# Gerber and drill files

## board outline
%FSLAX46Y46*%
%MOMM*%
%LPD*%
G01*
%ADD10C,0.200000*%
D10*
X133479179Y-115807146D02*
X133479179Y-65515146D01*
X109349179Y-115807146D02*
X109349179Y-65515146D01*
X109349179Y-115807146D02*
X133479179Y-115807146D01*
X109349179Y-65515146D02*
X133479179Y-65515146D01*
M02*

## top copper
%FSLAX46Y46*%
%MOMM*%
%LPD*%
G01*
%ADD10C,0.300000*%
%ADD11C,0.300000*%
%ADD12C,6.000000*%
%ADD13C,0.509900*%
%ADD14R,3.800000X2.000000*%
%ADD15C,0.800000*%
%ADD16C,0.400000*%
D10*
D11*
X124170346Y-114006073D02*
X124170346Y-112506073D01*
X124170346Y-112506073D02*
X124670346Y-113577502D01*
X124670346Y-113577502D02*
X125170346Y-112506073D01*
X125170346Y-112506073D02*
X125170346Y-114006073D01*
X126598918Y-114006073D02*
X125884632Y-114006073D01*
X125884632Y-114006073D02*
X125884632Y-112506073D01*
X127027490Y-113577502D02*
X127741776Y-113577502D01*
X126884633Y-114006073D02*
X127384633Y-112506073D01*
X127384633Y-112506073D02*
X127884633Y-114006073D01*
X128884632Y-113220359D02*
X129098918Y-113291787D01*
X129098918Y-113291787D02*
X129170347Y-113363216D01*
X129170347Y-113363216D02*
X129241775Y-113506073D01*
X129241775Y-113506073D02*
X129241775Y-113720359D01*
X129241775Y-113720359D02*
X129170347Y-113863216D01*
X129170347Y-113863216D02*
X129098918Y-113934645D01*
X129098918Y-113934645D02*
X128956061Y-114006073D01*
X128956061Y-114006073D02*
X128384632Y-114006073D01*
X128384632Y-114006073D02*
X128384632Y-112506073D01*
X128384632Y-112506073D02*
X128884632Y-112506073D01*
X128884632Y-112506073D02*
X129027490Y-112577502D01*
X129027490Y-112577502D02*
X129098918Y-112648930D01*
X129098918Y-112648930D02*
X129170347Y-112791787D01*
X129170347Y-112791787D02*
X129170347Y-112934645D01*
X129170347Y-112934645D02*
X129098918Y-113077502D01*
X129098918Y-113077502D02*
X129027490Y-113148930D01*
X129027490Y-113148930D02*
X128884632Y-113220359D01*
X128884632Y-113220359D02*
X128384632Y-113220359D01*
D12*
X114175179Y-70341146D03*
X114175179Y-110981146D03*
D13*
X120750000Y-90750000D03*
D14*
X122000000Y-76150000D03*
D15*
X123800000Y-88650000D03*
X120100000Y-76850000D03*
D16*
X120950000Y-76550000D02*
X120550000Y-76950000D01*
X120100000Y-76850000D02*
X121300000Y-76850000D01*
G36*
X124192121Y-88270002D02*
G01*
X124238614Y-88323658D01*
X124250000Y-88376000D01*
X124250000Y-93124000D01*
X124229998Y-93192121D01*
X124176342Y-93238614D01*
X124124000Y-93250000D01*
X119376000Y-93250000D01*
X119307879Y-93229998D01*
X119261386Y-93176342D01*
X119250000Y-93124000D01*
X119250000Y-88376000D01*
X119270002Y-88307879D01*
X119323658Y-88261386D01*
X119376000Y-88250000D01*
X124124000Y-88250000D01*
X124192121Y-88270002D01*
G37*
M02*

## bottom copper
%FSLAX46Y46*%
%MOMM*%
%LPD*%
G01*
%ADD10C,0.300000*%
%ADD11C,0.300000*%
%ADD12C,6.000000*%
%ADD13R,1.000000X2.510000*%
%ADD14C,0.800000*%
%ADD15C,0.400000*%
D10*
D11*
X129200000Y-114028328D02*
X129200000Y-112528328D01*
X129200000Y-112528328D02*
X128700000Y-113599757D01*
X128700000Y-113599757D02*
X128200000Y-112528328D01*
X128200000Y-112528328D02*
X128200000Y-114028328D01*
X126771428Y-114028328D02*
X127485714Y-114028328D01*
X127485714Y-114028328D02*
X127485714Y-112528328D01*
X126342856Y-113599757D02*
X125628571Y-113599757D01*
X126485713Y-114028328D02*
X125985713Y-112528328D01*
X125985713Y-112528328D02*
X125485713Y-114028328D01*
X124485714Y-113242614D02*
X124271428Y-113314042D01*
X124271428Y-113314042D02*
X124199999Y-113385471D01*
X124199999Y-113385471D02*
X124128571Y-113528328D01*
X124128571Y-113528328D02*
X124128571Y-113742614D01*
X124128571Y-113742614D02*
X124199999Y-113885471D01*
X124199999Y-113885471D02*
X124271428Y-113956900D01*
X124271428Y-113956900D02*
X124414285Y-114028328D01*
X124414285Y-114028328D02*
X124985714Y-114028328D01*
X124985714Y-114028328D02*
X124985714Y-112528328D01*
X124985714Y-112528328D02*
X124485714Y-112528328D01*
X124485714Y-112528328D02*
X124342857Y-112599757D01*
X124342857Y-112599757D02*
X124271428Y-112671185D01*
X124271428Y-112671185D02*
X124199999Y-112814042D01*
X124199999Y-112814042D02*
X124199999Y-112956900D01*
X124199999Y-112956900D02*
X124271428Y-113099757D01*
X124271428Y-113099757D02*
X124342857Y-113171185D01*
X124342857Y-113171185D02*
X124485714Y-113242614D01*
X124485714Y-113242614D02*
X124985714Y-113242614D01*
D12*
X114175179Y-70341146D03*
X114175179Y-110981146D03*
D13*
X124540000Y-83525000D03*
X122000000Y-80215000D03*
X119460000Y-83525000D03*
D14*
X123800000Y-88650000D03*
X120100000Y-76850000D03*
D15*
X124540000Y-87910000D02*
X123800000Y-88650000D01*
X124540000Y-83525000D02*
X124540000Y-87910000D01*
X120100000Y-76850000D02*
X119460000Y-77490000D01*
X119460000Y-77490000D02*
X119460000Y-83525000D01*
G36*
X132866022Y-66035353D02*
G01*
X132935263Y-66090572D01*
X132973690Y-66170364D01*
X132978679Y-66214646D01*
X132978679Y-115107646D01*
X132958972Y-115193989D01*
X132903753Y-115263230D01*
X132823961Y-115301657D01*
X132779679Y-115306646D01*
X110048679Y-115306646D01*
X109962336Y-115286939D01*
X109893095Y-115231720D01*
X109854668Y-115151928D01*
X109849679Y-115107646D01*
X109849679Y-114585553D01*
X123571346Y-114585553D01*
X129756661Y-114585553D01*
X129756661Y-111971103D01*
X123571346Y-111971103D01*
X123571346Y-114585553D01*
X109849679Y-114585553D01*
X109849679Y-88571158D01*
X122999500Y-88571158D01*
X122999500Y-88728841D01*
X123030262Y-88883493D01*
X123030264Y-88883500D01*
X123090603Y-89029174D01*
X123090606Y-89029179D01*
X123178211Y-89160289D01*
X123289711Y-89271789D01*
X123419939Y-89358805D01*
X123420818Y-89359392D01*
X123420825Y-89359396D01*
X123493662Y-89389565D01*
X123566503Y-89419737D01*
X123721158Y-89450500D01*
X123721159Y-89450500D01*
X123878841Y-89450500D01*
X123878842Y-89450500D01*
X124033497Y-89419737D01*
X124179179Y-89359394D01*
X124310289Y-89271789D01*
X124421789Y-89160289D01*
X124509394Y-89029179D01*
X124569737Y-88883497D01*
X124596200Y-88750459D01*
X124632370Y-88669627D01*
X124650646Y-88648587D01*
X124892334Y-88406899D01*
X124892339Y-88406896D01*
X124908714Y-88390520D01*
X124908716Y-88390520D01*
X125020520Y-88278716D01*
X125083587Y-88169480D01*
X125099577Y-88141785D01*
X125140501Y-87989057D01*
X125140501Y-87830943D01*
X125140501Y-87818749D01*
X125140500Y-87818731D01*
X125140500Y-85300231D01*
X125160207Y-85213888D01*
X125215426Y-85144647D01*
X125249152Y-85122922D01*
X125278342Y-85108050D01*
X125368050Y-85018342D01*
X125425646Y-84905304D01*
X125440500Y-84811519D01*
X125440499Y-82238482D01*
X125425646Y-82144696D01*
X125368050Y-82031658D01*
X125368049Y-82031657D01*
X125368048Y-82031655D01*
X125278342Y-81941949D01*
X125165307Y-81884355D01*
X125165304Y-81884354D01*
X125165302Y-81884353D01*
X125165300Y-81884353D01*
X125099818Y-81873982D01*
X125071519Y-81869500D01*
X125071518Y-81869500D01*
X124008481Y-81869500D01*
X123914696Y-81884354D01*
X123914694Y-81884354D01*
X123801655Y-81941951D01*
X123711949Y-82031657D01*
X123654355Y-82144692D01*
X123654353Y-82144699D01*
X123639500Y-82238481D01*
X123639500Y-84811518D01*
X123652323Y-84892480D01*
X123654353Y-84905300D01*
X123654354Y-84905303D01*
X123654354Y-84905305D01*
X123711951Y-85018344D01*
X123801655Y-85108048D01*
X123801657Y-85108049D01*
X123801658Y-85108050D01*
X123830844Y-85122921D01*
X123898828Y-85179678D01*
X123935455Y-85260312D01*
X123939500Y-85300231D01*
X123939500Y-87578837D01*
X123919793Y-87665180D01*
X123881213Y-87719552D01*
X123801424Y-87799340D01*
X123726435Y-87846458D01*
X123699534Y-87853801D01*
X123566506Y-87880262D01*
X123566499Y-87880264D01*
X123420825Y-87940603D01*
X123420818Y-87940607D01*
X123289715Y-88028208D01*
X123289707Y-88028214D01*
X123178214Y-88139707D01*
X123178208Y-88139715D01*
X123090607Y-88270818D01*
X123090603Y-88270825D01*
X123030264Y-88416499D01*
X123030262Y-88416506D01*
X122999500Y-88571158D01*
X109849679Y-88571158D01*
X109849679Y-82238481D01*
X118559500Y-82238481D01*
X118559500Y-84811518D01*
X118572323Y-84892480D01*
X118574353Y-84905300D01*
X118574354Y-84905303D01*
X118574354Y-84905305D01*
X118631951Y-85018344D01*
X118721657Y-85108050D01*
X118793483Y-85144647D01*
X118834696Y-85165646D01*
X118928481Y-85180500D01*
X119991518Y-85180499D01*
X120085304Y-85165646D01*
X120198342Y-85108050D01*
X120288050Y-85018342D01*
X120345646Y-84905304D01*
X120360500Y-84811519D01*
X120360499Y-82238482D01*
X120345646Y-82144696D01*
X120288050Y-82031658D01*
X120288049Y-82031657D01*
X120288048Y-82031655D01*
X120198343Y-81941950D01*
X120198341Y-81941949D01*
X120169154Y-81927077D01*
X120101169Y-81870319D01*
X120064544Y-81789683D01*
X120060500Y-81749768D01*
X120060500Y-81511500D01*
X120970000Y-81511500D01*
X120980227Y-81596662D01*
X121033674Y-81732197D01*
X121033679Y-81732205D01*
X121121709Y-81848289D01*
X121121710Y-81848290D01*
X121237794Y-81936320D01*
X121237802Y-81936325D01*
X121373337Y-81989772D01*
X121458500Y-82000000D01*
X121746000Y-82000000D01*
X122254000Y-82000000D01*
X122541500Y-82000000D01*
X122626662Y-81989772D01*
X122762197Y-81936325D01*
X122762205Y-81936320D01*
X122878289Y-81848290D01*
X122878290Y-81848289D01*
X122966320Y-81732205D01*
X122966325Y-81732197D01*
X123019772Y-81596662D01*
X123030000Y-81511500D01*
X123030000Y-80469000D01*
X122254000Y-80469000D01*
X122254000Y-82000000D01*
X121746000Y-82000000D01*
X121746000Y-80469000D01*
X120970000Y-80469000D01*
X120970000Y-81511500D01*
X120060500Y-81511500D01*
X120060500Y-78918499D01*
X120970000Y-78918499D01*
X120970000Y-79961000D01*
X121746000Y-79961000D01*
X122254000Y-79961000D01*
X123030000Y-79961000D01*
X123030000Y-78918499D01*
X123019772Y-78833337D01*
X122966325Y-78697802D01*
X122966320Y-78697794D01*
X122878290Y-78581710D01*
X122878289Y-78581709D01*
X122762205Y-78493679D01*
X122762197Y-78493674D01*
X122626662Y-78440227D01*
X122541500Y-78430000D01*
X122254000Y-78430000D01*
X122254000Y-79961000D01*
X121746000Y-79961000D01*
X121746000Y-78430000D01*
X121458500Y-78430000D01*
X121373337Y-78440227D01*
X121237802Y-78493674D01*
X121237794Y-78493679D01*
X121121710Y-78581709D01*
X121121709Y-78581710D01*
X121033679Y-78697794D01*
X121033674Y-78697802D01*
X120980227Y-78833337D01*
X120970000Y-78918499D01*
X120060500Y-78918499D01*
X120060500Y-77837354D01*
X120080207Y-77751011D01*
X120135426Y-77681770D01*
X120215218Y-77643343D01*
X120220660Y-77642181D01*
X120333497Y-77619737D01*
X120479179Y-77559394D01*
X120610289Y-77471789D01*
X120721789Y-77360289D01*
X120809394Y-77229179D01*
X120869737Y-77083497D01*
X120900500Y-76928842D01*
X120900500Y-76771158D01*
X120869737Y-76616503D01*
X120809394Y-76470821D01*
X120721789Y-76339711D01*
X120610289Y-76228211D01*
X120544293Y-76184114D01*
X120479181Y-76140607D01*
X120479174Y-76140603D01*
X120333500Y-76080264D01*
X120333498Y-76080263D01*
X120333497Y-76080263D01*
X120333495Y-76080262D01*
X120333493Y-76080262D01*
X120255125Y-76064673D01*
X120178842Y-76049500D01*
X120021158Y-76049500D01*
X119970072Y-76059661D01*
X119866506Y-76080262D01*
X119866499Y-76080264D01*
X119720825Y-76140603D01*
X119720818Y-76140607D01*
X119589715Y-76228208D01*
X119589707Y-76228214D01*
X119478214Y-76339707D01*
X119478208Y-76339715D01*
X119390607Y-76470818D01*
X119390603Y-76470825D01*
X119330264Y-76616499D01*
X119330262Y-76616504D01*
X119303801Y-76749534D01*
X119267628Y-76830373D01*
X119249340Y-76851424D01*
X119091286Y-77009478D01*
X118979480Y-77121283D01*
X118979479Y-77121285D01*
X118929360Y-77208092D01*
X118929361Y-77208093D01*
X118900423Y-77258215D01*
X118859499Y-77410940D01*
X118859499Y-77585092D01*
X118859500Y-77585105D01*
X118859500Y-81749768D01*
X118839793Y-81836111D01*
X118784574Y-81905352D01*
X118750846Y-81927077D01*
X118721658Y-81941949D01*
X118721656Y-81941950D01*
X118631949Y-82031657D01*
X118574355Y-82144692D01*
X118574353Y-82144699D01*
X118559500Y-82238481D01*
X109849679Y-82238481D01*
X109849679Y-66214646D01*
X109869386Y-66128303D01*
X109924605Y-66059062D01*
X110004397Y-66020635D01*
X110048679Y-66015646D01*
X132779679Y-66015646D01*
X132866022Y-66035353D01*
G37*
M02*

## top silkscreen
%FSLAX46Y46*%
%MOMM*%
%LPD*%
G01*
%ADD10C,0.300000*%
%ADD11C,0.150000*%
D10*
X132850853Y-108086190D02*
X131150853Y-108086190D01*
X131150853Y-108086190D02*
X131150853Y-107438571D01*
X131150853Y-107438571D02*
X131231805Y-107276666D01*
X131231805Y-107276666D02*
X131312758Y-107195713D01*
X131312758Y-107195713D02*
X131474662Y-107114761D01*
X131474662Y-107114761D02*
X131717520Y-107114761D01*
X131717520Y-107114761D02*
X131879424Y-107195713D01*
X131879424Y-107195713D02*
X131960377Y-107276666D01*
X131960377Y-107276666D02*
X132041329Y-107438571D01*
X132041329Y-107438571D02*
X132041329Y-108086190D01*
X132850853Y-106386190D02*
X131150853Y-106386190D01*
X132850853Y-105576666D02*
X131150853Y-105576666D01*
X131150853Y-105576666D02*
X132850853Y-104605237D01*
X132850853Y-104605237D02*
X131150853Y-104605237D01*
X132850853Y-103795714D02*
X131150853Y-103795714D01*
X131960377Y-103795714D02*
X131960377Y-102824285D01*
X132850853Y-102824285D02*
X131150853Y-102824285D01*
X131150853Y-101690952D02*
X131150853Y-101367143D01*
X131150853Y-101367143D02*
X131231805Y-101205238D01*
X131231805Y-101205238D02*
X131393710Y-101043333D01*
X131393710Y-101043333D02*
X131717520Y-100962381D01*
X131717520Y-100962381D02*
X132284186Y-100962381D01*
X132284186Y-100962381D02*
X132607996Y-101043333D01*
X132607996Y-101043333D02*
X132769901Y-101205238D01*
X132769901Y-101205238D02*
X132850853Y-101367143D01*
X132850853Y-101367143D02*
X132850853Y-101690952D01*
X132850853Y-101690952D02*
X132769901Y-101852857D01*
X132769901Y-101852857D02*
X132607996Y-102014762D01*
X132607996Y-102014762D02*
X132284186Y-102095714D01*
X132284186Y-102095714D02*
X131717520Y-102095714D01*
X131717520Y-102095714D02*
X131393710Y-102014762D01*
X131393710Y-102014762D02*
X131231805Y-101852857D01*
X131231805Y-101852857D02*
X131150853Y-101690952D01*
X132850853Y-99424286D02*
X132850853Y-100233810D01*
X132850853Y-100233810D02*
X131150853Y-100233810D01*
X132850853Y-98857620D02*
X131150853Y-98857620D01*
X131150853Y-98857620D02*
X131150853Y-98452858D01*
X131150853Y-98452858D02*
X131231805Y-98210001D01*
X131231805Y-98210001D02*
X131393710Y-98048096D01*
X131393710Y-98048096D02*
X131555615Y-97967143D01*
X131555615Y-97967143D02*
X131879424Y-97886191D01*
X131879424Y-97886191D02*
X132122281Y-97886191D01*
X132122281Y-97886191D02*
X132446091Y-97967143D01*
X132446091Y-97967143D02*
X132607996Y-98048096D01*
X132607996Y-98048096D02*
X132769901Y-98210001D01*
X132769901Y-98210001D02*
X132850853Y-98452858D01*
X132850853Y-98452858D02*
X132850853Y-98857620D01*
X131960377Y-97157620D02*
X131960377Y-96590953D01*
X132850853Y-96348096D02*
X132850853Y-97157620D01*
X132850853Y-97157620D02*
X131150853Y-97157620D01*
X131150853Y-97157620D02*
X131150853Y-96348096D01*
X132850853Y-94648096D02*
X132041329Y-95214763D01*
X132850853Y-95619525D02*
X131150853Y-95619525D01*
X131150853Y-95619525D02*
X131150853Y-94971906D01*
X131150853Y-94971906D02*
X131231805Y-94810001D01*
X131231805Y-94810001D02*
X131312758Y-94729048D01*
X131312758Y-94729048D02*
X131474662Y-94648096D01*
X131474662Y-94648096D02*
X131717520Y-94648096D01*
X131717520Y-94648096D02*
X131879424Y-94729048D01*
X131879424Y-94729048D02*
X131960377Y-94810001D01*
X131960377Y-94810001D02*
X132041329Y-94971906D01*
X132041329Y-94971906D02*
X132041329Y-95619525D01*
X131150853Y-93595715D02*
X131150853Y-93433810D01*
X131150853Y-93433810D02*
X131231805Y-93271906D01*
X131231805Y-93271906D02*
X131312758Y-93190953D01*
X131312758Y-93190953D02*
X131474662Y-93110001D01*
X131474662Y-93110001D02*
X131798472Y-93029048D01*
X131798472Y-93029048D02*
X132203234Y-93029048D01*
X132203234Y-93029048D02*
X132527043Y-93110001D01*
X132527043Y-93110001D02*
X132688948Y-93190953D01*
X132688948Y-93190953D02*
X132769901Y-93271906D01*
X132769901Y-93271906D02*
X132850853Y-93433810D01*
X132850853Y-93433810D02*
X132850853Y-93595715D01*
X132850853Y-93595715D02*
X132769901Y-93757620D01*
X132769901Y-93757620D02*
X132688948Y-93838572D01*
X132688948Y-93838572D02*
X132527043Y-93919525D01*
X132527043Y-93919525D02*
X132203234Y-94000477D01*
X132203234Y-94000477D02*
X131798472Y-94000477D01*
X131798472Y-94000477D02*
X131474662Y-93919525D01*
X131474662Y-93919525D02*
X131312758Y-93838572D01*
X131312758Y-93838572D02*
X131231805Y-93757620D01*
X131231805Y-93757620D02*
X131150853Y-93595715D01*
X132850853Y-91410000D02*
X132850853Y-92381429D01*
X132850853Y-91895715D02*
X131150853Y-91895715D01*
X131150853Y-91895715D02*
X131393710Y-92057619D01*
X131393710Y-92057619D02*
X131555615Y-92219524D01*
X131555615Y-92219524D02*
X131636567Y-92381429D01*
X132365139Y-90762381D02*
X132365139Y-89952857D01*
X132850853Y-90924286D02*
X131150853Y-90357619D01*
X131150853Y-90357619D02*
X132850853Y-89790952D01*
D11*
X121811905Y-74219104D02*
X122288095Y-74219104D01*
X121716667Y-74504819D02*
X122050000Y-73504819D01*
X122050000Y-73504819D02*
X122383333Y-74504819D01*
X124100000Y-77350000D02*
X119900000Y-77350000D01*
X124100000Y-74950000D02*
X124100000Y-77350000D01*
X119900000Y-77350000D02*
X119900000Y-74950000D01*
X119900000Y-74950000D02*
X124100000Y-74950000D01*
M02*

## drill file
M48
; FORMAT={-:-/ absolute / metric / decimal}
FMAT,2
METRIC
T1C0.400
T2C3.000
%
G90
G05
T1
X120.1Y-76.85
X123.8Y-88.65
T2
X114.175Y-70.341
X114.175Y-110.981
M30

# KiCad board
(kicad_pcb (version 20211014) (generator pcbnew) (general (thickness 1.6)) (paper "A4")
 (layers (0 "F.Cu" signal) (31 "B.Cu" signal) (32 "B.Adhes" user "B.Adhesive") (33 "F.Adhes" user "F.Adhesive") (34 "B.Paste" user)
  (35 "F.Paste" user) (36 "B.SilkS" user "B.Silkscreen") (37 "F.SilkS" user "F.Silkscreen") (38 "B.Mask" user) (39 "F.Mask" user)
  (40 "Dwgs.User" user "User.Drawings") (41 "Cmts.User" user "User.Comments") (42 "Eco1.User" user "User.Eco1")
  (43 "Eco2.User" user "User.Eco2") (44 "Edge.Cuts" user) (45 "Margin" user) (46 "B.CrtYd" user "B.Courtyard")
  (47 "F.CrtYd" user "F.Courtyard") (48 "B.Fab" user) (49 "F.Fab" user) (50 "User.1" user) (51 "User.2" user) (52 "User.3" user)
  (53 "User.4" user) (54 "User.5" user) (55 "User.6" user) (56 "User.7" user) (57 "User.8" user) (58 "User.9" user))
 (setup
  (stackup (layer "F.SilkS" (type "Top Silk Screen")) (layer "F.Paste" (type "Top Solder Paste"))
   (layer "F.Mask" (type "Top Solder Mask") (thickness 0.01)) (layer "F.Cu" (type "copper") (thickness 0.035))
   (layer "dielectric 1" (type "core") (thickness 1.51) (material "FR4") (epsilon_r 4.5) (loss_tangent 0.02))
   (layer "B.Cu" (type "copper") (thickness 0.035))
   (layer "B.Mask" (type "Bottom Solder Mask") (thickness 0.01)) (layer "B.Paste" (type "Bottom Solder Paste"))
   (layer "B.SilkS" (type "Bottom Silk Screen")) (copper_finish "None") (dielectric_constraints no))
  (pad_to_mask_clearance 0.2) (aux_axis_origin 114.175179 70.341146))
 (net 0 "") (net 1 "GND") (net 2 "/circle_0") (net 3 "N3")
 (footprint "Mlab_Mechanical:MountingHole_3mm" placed (layer "F.Cu") (at 114.175179 70.341146)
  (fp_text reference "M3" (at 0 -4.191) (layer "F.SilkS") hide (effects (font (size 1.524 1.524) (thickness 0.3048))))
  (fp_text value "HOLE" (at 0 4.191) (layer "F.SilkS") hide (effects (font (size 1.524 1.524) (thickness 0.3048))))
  (pad "1" thru_hole circle locked (at 0 0) (size 6 6) (drill 3) (layers F&B.Cu *.Adhes *.Mask) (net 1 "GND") (clearance 1) (zone_connect 2)))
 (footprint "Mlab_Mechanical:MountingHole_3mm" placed (layer "F.Cu") (at 114.175179 110.981146)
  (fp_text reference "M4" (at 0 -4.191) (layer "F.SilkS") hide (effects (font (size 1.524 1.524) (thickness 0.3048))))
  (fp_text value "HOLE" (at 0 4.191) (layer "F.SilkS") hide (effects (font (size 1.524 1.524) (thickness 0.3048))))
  (pad "1" thru_hole circle locked (at 0 0) (size 6 6) (drill 3) (layers F&B.Cu *.Adhes *.Mask) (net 1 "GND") (clearance 1) (zone_connect 2)))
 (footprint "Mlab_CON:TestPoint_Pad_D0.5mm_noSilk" (layer "F.Cu") (at 120.75 90.75 90) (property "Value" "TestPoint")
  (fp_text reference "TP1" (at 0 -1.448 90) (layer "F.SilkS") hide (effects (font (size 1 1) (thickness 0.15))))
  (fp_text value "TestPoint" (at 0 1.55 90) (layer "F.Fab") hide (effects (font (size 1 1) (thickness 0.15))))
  (pad "1" smd circle (at 0 0 90) (size 0.5099 0.5099) (layers "F.Cu" "F.Mask") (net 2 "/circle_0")))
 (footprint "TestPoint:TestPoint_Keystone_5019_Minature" (layer "F.Cu") (at 122 76.15 180) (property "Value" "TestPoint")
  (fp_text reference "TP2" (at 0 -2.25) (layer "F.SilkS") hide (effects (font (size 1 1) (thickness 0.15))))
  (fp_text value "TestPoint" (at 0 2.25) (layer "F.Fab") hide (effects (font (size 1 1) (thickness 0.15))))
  (fp_line (start -2.1 -1.2) (end 2.1 -1.2) (layer "F.SilkS") (width 0.15))
  (fp_line (start -2.1 1.2) (end -2.1 -1.2) (layer "F.SilkS") (width 0.15))
  (fp_line (start 2.1 -1.2) (end 2.1 1.2) (layer "F.SilkS") (width 0.15))
  (fp_line (start 2.1 1.2) (end -2.1 1.2) (layer "F.SilkS") (width 0.15))
  (pad "1" smd rect (at 0 0 180) (size 3.8 2) (layers "F.Cu" "F.Paste" "F.Mask") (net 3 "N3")))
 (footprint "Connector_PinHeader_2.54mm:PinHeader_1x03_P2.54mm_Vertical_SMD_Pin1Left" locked (layer "B.Cu") (at 122 81.87 90)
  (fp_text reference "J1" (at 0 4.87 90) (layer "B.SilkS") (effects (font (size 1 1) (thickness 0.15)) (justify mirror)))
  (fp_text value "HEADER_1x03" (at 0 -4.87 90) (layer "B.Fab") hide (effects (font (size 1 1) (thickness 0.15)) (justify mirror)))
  (pad "1" smd rect locked (at -1.655 2.54 90) (size 2.51 1) (layers "B.Cu" "B.Paste" "B.Mask") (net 2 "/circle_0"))
  (pad "2" smd rect locked (at 1.655 0 90) (size 2.51 1) (layers "B.Cu" "B.Paste" "B.Mask") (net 1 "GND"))
  (pad "3" smd rect locked (at -1.655 -2.54 90) (size 2.51 1) (layers "B.Cu" "B.Paste" "B.Mask") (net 3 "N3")))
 (gr_line (start 133.479179 115.807146) (end 133.479179 65.515146) (layer "Edge.Cuts") (width 0.2))
 (gr_line (start 109.349179 115.807146) (end 109.349179 65.515146) (layer "Edge.Cuts") (width 0.2))
 (gr_line (start 109.349179 115.807146) (end 133.479179 115.807146) (layer "Edge.Cuts") (width 0.2))
 (gr_line (start 109.349179 65.515146) (end 133.479179 65.515146) (layer "Edge.Cuts") (width 0.2))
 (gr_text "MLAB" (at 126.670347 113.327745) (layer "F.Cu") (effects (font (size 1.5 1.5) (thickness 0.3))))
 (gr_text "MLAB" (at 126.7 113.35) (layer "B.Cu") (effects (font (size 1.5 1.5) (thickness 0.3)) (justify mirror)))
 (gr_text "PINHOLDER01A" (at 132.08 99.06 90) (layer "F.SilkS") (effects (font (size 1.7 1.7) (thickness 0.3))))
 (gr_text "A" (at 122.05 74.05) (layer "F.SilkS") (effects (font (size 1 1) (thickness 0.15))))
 (via (at 123.8 88.65) (size 0.8) (drill 0.4) (layers "F.Cu" "B.Cu") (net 2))
 (segment (start 124.54 87.91) (end 123.8 88.65) (width 0.4) (layer "B.Cu") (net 2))
 (segment (start 124.54 83.525) (end 124.54 87.91) (width 0.4) (layer "B.Cu") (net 2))
 (segment (start 120.95 76.55) (end 120.55 76.95) (width 0.4) (layer "F.Cu") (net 3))
 (segment (start 120.1 76.85) (end 121.3 76.85) (width 0.4) (layer "F.Cu") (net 3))
 (via (at 120.1 76.85) (size 0.8) (drill 0.4) (layers "F.Cu" "B.Cu") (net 3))
 (segment (start 120.1 76.85) (end 119.46 77.49) (width 0.4) (layer "B.Cu") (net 3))
 (segment (start 119.46 77.49) (end 119.46 83.525) (width 0.4) (layer "B.Cu") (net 3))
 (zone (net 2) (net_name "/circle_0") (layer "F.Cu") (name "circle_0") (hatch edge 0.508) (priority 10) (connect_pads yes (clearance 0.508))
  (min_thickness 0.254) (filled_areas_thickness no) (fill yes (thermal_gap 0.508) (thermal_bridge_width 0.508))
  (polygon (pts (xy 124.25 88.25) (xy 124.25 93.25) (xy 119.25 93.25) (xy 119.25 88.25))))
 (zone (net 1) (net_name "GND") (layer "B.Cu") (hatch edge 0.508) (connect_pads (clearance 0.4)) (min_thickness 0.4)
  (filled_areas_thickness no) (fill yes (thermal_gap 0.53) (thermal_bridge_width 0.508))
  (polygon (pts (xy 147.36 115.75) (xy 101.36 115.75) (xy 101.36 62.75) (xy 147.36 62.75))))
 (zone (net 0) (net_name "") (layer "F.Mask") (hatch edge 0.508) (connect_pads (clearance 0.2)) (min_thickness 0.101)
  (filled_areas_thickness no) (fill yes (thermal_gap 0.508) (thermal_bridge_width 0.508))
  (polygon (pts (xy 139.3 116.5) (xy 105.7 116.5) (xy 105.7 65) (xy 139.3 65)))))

